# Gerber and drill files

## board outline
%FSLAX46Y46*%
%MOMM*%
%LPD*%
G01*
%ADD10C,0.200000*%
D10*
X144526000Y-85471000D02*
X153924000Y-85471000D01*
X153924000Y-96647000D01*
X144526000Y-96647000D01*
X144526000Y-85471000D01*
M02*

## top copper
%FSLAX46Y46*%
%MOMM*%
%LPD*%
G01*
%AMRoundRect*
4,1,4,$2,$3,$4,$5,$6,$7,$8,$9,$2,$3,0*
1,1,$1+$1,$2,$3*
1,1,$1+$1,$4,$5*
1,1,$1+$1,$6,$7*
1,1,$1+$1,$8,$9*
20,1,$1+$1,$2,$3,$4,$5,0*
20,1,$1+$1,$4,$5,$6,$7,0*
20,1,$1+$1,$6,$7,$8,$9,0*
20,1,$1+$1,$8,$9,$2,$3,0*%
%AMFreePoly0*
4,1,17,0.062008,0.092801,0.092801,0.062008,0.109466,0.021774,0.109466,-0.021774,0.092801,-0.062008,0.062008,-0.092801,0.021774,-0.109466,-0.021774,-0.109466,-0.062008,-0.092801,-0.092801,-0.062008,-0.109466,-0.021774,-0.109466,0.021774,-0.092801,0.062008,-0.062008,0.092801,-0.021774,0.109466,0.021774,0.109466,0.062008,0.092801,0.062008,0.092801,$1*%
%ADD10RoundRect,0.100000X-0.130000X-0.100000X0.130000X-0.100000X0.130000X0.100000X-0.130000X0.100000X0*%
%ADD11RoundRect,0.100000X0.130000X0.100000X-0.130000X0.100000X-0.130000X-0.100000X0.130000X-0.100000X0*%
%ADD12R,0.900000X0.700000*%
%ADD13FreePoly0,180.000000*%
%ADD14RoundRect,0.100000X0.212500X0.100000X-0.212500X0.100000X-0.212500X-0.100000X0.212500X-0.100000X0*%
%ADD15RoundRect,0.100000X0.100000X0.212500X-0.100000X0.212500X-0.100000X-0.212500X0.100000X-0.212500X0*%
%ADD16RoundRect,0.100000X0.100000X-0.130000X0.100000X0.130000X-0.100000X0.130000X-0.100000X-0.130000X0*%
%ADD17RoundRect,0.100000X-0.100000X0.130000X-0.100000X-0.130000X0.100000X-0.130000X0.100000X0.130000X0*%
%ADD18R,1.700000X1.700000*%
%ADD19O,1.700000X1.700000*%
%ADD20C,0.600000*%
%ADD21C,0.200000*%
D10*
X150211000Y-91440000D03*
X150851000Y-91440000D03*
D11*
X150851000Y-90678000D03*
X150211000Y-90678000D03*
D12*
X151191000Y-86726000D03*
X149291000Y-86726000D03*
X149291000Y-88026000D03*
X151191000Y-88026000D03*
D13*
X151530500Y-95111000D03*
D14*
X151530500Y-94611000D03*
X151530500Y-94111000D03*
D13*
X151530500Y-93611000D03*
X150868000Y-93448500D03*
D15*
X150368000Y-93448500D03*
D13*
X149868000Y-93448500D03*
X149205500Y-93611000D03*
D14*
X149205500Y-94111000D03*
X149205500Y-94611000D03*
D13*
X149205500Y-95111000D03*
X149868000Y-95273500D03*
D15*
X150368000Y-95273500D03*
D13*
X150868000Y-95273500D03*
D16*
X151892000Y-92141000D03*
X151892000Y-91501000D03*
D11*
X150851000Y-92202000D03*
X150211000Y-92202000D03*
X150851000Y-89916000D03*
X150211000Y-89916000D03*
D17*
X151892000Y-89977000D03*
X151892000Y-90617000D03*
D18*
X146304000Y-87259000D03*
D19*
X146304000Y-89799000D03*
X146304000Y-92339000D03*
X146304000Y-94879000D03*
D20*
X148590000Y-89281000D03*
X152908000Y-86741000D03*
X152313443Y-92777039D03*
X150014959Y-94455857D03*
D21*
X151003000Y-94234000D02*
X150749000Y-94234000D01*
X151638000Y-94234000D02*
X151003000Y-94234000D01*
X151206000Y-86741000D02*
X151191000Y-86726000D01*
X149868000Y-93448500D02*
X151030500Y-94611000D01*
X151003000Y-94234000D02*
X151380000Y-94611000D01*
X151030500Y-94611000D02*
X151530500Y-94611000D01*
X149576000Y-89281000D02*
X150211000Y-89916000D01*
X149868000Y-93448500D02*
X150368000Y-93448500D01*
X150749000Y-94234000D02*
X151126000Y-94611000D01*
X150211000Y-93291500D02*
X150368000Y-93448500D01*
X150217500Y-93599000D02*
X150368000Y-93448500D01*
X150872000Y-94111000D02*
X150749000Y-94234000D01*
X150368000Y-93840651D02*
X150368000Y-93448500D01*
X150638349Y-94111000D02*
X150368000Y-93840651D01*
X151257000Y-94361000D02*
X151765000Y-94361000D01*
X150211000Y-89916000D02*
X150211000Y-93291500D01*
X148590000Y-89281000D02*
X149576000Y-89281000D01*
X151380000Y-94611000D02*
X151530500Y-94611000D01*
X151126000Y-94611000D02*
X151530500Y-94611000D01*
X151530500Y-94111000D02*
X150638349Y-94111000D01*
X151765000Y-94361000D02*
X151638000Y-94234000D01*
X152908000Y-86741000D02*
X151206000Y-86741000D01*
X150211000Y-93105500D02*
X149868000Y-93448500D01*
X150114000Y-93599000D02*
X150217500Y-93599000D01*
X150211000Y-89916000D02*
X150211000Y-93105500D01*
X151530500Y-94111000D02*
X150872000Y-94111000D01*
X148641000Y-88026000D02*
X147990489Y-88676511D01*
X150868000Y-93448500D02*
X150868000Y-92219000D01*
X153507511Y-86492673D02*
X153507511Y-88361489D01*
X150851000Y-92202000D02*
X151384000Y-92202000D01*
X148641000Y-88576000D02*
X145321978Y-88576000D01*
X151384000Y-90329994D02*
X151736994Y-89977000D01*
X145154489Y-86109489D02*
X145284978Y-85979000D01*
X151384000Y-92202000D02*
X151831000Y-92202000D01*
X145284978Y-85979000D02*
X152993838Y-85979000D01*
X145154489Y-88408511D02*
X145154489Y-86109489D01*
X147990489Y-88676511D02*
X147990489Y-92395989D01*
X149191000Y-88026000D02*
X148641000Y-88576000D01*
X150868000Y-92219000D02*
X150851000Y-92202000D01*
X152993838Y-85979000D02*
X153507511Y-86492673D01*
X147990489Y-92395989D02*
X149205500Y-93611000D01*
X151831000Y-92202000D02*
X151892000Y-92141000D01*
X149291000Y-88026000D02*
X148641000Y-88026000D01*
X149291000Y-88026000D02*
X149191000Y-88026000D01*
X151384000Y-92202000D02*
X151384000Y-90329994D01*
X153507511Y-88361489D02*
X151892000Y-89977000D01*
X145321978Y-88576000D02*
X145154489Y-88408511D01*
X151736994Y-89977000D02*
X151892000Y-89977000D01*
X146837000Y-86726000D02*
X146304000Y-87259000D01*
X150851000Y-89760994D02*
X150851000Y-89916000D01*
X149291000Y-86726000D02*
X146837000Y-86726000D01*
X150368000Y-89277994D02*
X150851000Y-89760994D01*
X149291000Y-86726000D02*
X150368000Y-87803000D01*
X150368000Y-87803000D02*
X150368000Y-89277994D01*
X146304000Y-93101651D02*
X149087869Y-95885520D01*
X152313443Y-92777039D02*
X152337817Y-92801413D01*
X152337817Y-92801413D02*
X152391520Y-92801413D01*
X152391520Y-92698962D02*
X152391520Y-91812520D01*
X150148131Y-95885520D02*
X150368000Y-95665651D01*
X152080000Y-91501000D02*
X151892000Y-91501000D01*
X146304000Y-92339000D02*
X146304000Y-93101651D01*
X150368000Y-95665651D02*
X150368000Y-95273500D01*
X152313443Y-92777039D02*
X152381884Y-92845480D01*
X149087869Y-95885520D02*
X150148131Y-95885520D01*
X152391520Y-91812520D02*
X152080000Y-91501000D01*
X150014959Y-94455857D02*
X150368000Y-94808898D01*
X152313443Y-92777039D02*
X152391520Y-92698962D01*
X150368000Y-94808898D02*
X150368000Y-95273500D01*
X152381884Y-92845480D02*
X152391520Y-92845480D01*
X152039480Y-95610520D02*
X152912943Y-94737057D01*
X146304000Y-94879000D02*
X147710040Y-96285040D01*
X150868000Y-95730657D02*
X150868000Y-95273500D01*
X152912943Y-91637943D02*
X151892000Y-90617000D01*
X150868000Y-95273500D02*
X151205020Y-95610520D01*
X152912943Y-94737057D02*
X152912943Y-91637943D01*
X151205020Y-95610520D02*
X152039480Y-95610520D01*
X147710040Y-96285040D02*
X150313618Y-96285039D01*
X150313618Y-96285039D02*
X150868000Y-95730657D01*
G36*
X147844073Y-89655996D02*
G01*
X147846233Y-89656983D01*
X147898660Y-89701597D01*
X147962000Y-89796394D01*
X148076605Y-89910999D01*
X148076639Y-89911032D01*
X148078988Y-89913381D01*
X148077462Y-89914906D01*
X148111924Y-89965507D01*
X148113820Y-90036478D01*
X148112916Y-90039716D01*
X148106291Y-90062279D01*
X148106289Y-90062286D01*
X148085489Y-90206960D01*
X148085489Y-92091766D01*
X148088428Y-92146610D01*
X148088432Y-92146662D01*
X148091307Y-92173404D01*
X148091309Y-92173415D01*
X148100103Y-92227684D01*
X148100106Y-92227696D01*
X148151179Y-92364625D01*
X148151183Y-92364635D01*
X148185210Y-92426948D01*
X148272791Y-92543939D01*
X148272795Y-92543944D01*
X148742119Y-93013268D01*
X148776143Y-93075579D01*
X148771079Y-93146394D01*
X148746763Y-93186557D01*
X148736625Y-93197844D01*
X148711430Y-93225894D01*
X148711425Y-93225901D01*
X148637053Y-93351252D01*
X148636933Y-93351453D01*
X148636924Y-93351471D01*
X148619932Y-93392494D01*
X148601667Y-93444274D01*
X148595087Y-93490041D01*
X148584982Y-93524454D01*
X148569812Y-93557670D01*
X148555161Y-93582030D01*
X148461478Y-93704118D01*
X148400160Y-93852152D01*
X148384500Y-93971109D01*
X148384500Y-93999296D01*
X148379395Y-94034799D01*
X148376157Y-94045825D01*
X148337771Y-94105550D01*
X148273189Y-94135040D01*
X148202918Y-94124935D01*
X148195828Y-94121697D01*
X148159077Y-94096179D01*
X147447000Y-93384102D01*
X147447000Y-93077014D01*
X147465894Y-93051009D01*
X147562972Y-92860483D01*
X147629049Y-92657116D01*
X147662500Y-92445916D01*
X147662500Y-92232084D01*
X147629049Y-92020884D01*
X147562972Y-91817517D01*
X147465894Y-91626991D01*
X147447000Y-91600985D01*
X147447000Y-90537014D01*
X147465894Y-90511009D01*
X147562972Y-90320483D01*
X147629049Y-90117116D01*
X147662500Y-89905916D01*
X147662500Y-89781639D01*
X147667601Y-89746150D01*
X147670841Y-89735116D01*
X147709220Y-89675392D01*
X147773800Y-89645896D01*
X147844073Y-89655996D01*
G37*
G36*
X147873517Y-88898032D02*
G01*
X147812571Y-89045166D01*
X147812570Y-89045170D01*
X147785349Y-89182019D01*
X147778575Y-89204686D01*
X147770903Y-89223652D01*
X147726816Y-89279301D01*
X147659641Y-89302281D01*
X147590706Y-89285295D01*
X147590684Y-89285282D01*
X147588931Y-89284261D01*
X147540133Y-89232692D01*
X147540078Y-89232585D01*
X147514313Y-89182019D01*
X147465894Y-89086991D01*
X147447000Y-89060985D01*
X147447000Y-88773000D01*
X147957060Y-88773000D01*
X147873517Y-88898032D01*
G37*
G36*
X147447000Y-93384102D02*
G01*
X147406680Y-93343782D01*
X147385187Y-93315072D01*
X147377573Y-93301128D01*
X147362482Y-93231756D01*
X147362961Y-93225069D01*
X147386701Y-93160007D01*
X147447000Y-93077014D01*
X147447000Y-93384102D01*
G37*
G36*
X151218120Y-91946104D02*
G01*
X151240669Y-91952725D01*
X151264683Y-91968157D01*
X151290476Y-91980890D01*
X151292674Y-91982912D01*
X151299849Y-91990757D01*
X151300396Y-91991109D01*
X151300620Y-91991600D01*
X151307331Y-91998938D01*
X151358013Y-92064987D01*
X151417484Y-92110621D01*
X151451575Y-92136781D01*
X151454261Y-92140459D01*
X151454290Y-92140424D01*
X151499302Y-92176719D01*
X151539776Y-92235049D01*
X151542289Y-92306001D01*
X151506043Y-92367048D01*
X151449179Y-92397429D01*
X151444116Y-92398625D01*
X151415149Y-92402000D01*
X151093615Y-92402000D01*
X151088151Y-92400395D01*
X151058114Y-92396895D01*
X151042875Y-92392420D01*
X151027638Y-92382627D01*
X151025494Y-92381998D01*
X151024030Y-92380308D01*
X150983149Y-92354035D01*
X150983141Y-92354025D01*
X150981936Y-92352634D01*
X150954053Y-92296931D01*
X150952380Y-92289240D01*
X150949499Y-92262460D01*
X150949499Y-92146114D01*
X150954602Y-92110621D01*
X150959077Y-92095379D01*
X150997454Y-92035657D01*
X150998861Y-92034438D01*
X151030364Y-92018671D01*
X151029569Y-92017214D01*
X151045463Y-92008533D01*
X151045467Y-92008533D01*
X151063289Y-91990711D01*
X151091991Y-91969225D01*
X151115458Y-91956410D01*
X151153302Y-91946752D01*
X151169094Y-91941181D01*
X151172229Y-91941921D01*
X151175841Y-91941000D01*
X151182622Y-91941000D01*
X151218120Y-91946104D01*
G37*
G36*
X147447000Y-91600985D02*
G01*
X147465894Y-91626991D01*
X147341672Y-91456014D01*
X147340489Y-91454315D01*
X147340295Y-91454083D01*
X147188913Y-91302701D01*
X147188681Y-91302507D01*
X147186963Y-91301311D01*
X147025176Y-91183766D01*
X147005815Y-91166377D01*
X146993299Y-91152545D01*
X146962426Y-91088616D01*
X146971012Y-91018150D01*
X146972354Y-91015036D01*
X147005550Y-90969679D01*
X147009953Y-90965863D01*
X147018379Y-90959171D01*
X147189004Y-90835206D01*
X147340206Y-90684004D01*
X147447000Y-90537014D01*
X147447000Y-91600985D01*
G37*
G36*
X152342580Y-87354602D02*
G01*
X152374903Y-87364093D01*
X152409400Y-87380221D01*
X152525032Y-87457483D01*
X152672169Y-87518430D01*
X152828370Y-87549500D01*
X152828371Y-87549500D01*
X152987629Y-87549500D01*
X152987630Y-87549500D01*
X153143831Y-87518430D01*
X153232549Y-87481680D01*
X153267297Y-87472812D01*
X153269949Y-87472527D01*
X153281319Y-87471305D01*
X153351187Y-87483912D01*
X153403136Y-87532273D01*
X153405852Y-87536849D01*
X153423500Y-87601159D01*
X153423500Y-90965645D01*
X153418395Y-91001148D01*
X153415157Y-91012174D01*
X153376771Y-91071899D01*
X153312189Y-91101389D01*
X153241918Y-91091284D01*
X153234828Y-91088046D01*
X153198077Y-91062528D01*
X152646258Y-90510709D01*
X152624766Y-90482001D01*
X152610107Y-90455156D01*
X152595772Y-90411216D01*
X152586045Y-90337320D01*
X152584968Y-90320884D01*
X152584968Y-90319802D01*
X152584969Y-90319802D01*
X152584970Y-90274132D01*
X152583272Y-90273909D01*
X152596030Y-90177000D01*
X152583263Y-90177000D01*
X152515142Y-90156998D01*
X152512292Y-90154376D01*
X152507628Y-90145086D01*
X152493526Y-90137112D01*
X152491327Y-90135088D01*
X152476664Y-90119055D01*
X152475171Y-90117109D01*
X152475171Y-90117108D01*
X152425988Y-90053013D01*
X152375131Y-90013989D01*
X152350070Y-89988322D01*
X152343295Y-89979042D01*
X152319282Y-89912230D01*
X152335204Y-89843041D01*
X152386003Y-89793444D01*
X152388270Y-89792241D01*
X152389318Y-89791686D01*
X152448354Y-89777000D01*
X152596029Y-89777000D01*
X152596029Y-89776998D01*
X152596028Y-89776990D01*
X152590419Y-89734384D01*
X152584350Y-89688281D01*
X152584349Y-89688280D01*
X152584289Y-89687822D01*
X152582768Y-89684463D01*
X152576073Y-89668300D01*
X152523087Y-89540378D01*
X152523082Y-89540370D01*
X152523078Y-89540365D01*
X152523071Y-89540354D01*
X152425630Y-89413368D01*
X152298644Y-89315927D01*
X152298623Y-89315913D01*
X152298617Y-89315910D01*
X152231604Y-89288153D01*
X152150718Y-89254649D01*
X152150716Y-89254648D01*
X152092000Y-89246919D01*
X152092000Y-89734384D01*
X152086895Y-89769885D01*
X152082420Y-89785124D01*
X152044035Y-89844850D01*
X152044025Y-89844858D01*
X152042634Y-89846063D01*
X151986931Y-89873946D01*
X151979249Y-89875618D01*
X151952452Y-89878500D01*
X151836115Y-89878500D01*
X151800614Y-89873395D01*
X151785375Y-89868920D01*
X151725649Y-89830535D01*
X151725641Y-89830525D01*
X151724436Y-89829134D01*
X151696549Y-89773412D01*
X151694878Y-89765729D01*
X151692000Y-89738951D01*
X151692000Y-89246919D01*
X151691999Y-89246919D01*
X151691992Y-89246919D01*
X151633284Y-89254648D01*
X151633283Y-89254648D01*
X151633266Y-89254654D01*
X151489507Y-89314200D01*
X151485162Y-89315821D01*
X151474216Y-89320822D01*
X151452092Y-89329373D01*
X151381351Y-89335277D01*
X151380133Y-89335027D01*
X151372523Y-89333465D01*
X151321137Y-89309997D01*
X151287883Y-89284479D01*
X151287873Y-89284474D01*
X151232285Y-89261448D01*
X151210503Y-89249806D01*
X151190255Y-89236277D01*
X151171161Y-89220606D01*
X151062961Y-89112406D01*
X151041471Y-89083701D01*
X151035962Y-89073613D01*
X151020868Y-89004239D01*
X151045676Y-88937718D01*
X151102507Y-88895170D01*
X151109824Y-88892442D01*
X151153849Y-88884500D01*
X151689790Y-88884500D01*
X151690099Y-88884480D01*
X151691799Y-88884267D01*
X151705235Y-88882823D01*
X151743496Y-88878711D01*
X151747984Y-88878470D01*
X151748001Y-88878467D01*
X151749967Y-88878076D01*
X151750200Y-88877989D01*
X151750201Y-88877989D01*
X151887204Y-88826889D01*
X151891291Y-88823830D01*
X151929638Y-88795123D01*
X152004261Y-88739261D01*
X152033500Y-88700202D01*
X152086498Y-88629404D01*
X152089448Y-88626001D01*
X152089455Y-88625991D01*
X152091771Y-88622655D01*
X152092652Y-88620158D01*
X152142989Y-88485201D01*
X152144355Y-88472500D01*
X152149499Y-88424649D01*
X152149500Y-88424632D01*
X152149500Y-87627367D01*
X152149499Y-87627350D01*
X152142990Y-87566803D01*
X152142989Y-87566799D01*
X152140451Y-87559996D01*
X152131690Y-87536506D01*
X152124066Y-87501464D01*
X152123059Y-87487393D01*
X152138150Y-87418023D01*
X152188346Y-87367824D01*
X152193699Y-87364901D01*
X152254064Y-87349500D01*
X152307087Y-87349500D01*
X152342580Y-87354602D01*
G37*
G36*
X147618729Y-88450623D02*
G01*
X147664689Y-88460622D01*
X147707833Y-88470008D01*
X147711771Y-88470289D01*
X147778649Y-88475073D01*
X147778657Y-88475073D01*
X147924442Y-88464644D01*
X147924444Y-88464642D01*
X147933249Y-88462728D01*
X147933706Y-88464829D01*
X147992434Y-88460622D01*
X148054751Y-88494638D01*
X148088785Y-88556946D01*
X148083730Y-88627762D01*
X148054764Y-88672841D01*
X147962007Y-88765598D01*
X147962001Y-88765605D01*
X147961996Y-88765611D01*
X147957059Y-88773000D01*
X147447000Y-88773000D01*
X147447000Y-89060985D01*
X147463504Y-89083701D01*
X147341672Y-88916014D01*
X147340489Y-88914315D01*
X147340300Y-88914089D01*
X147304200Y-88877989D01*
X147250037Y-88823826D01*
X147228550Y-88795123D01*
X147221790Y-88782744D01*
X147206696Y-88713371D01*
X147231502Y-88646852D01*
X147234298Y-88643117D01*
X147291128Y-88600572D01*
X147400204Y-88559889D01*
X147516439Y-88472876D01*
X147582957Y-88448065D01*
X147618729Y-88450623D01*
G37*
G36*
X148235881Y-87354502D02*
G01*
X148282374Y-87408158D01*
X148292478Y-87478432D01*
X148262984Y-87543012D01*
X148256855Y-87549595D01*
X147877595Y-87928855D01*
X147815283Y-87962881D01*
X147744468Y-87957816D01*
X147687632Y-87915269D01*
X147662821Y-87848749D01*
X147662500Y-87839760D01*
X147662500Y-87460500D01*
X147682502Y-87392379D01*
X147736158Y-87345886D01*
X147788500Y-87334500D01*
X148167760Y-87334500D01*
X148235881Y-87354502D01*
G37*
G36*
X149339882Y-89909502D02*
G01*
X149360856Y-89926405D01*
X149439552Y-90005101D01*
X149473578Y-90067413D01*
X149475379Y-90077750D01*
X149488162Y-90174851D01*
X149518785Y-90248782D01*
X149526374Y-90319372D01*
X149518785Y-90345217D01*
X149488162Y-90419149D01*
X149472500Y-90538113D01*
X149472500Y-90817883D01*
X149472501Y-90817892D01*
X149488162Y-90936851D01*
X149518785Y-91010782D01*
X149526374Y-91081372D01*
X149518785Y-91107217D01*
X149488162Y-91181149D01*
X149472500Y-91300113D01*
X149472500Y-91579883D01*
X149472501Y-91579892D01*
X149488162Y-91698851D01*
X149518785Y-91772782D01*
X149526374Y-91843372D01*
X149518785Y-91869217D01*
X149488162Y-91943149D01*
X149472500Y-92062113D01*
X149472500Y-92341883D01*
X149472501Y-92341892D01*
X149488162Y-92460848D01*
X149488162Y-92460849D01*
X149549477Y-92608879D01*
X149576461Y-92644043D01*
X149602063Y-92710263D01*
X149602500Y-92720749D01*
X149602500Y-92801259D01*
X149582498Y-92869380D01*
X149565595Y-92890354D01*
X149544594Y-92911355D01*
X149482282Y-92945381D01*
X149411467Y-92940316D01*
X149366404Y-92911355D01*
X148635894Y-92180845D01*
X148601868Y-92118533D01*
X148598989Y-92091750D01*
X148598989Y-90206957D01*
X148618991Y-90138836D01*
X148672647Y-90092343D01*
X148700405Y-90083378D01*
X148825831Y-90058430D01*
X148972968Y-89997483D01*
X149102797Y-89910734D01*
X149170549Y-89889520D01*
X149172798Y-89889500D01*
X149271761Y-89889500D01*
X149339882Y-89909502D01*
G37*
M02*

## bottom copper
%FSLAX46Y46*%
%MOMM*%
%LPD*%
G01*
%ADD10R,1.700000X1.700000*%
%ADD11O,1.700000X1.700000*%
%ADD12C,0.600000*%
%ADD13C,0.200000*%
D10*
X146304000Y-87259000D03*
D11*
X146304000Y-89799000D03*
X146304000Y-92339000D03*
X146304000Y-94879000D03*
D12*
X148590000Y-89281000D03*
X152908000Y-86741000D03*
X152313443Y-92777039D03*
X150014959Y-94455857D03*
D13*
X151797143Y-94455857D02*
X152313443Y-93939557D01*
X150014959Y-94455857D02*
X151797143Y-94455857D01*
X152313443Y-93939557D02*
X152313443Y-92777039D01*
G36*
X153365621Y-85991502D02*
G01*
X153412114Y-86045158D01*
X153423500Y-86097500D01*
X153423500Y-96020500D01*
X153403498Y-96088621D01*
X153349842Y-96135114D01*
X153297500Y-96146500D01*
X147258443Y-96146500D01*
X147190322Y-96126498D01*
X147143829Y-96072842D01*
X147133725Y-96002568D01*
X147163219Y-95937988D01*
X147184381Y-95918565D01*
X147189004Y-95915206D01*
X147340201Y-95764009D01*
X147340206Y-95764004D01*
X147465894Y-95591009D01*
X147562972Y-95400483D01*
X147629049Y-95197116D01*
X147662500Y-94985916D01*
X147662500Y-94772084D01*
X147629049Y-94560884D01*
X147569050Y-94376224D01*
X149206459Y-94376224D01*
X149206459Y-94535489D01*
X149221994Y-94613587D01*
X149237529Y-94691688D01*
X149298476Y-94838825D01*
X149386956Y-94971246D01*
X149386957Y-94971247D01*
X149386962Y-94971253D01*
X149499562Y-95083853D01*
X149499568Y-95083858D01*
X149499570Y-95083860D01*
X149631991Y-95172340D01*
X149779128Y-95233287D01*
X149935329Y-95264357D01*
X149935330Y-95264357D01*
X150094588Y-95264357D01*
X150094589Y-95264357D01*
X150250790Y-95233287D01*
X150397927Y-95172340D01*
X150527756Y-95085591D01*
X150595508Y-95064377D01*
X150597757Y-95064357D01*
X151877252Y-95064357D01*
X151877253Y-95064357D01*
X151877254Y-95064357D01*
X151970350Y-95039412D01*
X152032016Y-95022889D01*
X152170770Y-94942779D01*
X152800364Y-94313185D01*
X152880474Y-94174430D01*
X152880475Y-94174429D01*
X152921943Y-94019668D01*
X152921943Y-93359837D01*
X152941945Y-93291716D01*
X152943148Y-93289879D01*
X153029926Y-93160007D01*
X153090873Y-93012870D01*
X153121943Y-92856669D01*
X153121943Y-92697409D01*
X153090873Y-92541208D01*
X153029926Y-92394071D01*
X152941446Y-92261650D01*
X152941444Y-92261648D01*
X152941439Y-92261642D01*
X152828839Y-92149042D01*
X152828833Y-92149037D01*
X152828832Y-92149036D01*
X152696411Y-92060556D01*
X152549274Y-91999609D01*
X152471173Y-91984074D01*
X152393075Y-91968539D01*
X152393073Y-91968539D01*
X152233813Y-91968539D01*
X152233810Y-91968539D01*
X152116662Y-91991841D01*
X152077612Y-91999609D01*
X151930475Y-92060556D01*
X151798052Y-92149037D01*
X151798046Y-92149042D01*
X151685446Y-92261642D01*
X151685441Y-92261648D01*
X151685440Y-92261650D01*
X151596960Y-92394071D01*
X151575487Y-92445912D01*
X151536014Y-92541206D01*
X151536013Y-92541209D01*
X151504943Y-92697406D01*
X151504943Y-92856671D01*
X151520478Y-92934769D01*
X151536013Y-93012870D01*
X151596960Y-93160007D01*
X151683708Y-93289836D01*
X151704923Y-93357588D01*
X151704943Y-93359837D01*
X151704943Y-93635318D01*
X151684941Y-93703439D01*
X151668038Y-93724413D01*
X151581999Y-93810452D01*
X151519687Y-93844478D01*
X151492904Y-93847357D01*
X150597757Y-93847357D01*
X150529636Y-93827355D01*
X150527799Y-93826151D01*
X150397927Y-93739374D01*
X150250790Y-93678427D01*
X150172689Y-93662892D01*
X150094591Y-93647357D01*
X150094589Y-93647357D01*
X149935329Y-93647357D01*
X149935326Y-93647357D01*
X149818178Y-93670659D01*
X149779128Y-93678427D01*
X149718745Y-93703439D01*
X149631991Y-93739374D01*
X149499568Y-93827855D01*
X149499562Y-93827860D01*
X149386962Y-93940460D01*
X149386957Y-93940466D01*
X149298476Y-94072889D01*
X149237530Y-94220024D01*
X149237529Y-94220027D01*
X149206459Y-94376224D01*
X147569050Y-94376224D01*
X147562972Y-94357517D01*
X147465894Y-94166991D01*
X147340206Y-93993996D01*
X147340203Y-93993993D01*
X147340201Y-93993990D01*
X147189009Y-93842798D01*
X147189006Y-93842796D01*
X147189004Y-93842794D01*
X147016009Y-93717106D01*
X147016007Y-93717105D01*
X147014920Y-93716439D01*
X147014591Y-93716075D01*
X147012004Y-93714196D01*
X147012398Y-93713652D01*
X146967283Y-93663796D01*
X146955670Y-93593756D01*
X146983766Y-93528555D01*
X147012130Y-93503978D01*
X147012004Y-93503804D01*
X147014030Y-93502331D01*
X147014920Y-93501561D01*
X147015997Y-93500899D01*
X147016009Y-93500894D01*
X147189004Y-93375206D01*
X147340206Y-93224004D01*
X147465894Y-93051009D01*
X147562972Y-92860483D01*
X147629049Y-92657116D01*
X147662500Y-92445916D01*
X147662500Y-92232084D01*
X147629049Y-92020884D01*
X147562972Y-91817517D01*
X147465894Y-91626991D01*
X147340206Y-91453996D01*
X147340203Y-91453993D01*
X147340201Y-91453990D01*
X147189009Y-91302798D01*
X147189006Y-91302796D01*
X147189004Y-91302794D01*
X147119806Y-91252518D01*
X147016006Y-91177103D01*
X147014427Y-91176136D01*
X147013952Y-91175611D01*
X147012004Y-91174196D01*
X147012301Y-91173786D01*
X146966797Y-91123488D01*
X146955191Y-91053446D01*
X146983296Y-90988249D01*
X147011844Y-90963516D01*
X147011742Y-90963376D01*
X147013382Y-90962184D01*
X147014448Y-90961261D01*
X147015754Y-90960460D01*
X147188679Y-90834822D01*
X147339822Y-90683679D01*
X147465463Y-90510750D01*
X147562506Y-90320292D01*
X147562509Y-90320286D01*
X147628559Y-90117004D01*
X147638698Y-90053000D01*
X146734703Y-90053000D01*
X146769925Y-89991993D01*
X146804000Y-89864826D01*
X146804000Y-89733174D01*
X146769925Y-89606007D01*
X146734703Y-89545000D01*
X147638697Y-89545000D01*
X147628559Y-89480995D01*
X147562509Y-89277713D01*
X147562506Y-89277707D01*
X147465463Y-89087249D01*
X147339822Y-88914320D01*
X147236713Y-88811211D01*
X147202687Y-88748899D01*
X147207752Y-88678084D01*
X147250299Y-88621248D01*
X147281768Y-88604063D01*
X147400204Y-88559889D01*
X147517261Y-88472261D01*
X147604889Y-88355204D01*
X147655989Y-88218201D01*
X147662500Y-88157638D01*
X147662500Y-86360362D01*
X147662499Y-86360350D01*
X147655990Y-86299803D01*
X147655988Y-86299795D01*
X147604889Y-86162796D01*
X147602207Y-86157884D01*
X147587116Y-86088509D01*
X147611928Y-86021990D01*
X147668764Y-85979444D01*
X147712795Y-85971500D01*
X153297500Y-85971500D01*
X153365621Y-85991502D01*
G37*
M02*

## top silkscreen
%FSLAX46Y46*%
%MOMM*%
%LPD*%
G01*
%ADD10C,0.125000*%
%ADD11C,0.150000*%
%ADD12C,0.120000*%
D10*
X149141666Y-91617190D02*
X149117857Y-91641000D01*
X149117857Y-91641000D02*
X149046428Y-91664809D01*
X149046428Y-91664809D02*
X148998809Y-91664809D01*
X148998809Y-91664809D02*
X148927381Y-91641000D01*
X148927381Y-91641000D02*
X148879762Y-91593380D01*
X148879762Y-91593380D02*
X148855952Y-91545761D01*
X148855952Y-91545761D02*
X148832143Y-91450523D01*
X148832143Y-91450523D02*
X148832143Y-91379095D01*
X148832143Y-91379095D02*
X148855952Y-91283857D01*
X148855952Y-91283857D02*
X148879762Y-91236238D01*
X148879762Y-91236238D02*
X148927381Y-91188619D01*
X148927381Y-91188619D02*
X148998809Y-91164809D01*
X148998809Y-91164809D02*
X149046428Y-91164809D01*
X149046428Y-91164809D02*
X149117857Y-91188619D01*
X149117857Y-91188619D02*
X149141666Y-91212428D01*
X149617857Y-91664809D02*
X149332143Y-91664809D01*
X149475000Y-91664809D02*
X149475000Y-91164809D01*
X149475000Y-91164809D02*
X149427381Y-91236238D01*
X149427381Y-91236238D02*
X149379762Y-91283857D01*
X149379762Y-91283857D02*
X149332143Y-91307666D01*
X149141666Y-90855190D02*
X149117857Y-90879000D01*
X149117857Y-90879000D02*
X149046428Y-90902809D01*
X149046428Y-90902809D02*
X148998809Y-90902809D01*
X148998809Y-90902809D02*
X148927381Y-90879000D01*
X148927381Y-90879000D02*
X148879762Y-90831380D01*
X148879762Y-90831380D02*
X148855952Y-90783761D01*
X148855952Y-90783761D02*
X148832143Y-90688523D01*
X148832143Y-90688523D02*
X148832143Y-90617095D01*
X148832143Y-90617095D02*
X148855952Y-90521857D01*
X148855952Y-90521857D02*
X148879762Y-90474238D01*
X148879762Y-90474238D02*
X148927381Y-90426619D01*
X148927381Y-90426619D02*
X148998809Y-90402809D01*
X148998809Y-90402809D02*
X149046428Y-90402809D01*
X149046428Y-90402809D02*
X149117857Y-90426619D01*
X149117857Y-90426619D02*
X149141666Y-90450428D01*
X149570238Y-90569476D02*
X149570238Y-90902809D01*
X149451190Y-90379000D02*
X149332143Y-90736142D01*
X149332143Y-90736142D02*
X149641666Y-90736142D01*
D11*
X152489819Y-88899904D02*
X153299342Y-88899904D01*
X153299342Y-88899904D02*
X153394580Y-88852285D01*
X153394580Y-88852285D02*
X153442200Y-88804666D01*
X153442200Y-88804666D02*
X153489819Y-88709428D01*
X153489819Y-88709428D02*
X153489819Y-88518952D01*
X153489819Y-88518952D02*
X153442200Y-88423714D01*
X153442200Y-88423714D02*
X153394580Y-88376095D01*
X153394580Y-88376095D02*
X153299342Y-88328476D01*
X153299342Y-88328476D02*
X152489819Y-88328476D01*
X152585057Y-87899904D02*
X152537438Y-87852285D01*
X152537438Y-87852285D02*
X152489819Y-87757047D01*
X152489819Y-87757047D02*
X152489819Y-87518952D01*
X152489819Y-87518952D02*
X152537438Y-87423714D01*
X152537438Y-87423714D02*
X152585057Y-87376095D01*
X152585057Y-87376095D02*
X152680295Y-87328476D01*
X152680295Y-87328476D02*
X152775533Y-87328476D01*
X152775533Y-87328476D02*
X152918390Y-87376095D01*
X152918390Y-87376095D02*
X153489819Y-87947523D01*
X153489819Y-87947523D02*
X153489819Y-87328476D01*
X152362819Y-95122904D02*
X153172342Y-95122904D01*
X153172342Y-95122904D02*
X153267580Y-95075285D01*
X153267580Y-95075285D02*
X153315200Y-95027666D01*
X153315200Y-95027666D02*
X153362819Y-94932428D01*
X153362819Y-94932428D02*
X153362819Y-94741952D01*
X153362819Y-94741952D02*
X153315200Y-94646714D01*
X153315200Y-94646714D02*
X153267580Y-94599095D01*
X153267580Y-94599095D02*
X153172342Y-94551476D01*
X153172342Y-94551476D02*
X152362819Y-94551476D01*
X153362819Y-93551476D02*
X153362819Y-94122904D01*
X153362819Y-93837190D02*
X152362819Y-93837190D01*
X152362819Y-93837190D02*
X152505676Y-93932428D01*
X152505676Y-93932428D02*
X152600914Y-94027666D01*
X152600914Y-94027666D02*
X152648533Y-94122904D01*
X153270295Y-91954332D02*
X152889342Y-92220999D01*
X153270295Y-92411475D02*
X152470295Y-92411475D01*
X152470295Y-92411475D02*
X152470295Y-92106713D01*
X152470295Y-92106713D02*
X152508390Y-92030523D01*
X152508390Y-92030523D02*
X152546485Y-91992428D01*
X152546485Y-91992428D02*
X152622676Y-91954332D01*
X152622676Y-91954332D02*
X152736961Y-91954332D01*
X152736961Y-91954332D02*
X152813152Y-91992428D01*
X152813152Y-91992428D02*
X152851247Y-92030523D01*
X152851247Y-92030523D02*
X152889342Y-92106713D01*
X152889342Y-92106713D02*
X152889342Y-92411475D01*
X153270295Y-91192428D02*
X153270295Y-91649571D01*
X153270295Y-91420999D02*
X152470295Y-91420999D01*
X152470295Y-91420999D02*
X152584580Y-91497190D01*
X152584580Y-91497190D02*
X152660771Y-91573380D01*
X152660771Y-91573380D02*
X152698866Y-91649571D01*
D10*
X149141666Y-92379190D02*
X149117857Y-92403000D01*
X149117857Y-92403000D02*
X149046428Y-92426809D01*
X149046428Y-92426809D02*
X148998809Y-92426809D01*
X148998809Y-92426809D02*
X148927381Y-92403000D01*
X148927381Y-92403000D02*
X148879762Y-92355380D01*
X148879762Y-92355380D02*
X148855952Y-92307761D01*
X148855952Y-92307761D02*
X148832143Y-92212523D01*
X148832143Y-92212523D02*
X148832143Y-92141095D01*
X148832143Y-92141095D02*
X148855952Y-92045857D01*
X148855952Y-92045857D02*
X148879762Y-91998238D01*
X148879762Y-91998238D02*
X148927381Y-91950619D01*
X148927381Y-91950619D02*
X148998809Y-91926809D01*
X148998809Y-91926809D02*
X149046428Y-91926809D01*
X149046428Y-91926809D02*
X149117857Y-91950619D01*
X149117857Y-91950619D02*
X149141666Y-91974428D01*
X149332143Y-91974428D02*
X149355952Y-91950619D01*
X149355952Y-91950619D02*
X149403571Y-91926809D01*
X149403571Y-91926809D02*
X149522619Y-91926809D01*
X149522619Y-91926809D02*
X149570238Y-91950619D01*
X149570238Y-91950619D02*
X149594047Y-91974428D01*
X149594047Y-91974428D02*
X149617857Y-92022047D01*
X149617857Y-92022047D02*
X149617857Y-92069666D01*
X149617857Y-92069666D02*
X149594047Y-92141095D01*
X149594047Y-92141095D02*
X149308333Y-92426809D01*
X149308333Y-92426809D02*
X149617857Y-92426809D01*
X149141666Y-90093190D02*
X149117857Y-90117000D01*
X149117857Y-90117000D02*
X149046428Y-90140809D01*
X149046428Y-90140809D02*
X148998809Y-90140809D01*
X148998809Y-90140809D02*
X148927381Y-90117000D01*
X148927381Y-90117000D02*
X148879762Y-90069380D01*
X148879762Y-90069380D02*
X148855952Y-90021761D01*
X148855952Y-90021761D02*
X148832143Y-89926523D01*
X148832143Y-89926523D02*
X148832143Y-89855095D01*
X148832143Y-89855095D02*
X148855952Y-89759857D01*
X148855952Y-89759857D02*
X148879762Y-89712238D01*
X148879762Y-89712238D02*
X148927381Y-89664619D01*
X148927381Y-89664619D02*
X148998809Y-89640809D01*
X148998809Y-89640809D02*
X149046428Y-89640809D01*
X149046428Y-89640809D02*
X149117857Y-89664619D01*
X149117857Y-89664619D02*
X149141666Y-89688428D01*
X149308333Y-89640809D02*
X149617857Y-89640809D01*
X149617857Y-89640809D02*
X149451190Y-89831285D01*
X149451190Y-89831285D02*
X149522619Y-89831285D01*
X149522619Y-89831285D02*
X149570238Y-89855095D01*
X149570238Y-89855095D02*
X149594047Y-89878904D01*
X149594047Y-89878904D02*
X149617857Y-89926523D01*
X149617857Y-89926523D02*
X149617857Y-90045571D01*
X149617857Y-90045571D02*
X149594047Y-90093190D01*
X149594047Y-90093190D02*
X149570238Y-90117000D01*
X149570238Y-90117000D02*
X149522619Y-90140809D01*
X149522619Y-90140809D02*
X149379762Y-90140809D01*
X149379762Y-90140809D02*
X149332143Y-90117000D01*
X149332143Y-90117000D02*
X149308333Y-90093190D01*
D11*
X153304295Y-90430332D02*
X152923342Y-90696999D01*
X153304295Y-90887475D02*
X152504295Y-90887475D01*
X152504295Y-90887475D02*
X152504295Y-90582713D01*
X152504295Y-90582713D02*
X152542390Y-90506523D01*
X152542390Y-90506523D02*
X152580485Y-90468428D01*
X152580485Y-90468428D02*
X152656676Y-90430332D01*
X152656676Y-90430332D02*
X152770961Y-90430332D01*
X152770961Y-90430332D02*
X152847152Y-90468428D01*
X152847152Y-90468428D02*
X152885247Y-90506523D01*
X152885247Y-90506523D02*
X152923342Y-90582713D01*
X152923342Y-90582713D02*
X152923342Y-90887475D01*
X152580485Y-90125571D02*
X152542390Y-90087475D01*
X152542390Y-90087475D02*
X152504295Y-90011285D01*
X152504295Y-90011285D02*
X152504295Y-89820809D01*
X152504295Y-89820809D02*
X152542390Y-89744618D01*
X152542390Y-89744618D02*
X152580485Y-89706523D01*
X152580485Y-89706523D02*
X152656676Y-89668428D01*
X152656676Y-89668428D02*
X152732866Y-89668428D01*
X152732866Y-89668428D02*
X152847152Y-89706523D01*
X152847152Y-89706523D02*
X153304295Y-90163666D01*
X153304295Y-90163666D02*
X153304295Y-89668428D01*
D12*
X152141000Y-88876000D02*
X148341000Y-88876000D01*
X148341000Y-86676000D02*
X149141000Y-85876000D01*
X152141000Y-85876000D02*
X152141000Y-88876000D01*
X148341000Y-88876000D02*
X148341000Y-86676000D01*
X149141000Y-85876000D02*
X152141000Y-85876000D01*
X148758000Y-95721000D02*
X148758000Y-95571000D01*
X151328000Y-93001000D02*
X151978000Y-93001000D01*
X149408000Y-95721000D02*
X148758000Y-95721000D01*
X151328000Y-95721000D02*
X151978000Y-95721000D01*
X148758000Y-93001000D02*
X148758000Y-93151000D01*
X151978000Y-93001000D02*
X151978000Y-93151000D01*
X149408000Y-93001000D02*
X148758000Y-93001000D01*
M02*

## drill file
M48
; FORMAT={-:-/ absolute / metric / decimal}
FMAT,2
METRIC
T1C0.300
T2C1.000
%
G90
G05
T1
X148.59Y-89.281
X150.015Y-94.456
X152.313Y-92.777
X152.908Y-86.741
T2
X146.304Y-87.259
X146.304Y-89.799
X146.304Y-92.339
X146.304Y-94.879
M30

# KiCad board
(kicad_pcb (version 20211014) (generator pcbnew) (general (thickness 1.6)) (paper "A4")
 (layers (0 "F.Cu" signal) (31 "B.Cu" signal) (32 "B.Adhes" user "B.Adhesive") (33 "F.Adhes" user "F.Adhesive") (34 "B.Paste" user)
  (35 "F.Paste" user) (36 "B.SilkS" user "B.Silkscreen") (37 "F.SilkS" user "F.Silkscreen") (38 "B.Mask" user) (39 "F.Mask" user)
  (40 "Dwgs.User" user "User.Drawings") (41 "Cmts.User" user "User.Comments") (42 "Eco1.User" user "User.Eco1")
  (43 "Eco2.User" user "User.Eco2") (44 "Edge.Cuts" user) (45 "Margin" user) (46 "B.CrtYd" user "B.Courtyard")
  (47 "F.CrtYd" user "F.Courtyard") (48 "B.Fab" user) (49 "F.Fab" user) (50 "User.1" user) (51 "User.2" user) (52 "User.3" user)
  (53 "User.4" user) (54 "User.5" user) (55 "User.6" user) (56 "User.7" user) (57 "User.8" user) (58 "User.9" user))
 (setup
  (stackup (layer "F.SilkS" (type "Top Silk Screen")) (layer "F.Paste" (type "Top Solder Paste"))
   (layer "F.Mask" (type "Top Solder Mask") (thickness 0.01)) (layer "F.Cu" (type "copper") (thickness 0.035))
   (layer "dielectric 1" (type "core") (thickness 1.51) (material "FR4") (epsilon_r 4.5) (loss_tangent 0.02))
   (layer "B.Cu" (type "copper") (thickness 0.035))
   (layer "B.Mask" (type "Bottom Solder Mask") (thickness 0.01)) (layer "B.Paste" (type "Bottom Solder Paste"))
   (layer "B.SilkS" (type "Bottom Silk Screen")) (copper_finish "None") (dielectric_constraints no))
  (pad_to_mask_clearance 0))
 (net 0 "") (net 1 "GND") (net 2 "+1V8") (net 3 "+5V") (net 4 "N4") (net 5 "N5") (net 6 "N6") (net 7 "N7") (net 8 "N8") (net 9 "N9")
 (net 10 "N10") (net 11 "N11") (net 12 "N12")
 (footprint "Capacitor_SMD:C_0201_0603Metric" (layer "F.Cu") (at 150.531 91.44)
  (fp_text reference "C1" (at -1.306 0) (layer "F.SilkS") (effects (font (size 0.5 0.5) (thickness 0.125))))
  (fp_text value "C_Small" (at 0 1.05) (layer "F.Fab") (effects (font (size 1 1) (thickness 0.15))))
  (pad "" smd roundrect (at -0.345 0) (size 0.318 0.36) (layers "F.Paste") (roundrect_rratio 0.25))
  (pad "" smd roundrect (at 0.345 0) (size 0.318 0.36) (layers "F.Paste") (roundrect_rratio 0.25))
  (pad "1" smd roundrect (at -0.32 0) (size 0.46 0.4) (layers "F.Cu" "F.Mask") (roundrect_rratio 0.25) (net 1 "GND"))
  (pad "2" smd roundrect (at 0.32 0) (size 0.46 0.4) (layers "F.Cu" "F.Mask") (roundrect_rratio 0.25) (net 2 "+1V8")))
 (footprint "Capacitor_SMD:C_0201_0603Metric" (layer "F.Cu") (at 150.531 90.678 180)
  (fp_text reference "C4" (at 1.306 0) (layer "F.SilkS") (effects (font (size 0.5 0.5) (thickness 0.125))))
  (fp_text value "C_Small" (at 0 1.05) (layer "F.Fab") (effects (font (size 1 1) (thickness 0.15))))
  (pad "" smd roundrect (at -0.345 0 180) (size 0.318 0.36) (layers "F.Paste") (roundrect_rratio 0.25))
  (pad "" smd roundrect (at 0.345 0 180) (size 0.318 0.36) (layers "F.Paste") (roundrect_rratio 0.25))
  (pad "1" smd roundrect (at -0.32 0 180) (size 0.46 0.4) (layers "F.Cu" "F.Mask") (roundrect_rratio 0.25) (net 2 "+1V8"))
  (pad "2" smd roundrect (at 0.32 0 180) (size 0.46 0.4) (layers "F.Cu" "F.Mask") (roundrect_rratio 0.25) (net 1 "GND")))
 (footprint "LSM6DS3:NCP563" (layer "F.Cu") (at 150.241 87.376 -90)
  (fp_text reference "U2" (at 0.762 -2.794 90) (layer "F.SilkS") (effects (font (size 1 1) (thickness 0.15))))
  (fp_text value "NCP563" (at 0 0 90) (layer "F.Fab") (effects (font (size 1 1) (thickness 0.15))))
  (fp_line (start 1.5 -1.9) (end 1.5 1.9) (layer "F.SilkS") (width 0.12))
  (fp_line (start -0.7 1.9) (end -1.5 1.1) (layer "F.SilkS") (width 0.12))
  (fp_line (start -1.5 -1.9) (end 1.5 -1.9) (layer "F.SilkS") (width 0.12))
  (fp_line (start 1.5 1.9) (end -0.7 1.9) (layer "F.SilkS") (width 0.12))
  (fp_line (start -1.5 1.1) (end -1.5 -1.9) (layer "F.SilkS") (width 0.12))
  (pad "1" smd rect (at -0.65 -0.95 270) (size 0.7 0.9) (layers "F.Cu" "F.Paste" "F.Mask") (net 1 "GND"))
  (pad "2" smd rect (at -0.65 0.95 270) (size 0.7 0.9) (layers "F.Cu" "F.Paste" "F.Mask") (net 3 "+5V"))
  (pad "3" smd rect (at 0.65 0.95 270) (size 0.7 0.9) (layers "F.Cu" "F.Paste" "F.Mask") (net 2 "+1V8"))
  (pad "4" smd rect (at 0.65 -0.95 270) (size 0.7 0.9) (layers "F.Cu" "F.Paste" "F.Mask") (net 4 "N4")))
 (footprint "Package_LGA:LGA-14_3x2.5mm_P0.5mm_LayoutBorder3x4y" (layer "F.Cu") (at 150.368 94.361 180)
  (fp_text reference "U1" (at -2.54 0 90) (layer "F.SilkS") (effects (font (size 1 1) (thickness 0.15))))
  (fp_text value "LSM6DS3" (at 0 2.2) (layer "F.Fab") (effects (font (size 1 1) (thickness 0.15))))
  (fp_line (start 1.61 -1.36) (end 1.61 -1.21) (layer "F.SilkS") (width 0.12))
  (fp_line (start -0.96 1.36) (end -1.61 1.36) (layer "F.SilkS") (width 0.12))
  (fp_line (start 0.96 -1.36) (end 1.61 -1.36) (layer "F.SilkS") (width 0.12))
  (fp_line (start -0.96 -1.36) (end -1.61 -1.36) (layer "F.SilkS") (width 0.12))
  (fp_line (start 1.61 1.36) (end 1.61 1.21) (layer "F.SilkS") (width 0.12))
  (fp_line (start -1.61 1.36) (end -1.61 1.21) (layer "F.SilkS") (width 0.12))
  (fp_line (start 0.96 1.36) (end 1.61 1.36) (layer "F.SilkS") (width 0.12))
  (pad "1" smd custom (at -1.1625 -0.75 180) (size 0.223223 0.223223) (layers "F.Cu" "F.Paste" "F.Mask") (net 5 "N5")
   (options (clearance outline) (anchor circle)) (primitives))
  (pad "2" smd roundrect (at -1.1625 -0.25 180) (size 0.625 0.4) (layers "F.Cu" "F.Paste" "F.Mask") (roundrect_rratio 0.25) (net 1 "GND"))
  (pad "3" smd roundrect (at -1.1625 0.25 180) (size 0.625 0.4) (layers "F.Cu" "F.Paste" "F.Mask") (roundrect_rratio 0.25) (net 1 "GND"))
  (pad "4" smd custom (at -1.1625 0.75 180) (size 0.223223 0.223223) (layers "F.Cu" "F.Paste" "F.Mask") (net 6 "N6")
   (options (clearance outline) (anchor circle)) (primitives))
  (pad "5" smd custom (at -0.5 0.9125 180) (size 0.223223 0.223223) (layers "F.Cu" "F.Paste" "F.Mask") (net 2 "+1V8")
   (options (clearance outline) (anchor circle)) (primitives))
  (pad "6" smd roundrect (at 0 0.9125 180) (size 0.4 0.625) (layers "F.Cu" "F.Paste" "F.Mask") (roundrect_rratio 0.25) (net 1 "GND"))
  (pad "7" smd custom (at 0.5 0.9125 180) (size 0.223223 0.223223) (layers "F.Cu" "F.Paste" "F.Mask") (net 1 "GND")
   (options (clearance outline) (anchor circle)) (primitives))
  (pad "8" smd custom (at 1.1625 0.75 180) (size 0.223223 0.223223) (layers "F.Cu" "F.Paste" "F.Mask") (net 2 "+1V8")
   (options (clearance outline) (anchor circle)) (primitives))
  (pad "9" smd roundrect (at 1.1625 0.25 180) (size 0.625 0.4) (layers "F.Cu" "F.Paste" "F.Mask") (roundrect_rratio 0.25) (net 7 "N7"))
  (pad "10" smd roundrect (at 1.1625 -0.25 180) (size 0.625 0.4) (layers "F.Cu" "F.Paste" "F.Mask") (roundrect_rratio 0.25) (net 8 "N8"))
  (pad "11" smd custom (at 1.1625 -0.75 180) (size 0.223223 0.223223) (layers "F.Cu" "F.Paste" "F.Mask") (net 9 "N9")
   (options (clearance outline) (anchor circle)) (primitives))
  (pad "12" smd custom (at 0.5 -0.9125 180) (size 0.223223 0.223223) (layers "F.Cu" "F.Paste" "F.Mask") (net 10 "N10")
   (options (clearance outline) (anchor circle)) (primitives))
  (pad "13" smd roundrect (at 0 -0.9125 180) (size 0.4 0.625) (layers "F.Cu" "F.Paste" "F.Mask") (roundrect_rratio 0.25) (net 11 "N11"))
  (pad "14" smd custom (at -0.5 -0.9125 180) (size 0.223223 0.223223) (layers "F.Cu" "F.Paste" "F.Mask") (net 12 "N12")
   (options (clearance outline) (anchor circle)) (primitives)))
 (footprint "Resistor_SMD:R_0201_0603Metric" (layer "F.Cu") (at 151.892 91.821 90)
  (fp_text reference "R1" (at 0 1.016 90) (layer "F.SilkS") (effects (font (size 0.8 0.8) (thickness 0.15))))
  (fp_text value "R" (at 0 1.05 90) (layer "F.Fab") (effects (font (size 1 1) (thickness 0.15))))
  (pad "" smd roundrect (at -0.345 0 90) (size 0.318 0.36) (layers "F.Paste") (roundrect_rratio 0.25))
  (pad "" smd roundrect (at 0.345 0 90) (size 0.318 0.36) (layers "F.Paste") (roundrect_rratio 0.25))
  (pad "1" smd roundrect (at -0.32 0 90) (size 0.46 0.4) (layers "F.Cu" "F.Mask") (roundrect_rratio 0.25) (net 2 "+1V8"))
  (pad "2" smd roundrect (at 0.32 0 90) (size 0.46 0.4) (layers "F.Cu" "F.Mask") (roundrect_rratio 0.25) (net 11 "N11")))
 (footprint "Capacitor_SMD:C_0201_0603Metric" (layer "F.Cu") (at 150.531 92.202 180)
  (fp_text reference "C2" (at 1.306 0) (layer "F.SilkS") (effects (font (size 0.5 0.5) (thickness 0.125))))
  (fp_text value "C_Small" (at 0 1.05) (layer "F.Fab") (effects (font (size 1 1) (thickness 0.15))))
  (pad "" smd roundrect (at 0.345 0 180) (size 0.318 0.36) (layers "F.Paste") (roundrect_rratio 0.25))
  (pad "" smd roundrect (at -0.345 0 180) (size 0.318 0.36) (layers "F.Paste") (roundrect_rratio 0.25))
  (pad "1" smd roundrect (at -0.32 0 180) (size 0.46 0.4) (layers "F.Cu" "F.Mask") (roundrect_rratio 0.25) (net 2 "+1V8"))
  (pad "2" smd roundrect (at 0.32 0 180) (size 0.46 0.4) (layers "F.Cu" "F.Mask") (roundrect_rratio 0.25) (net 1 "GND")))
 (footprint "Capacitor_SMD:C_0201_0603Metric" (layer "F.Cu") (at 150.531 89.916 180)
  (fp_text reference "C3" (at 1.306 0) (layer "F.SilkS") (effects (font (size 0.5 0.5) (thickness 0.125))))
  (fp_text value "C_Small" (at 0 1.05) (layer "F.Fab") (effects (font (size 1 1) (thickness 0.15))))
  (pad "" smd roundrect (at -0.345 0 180) (size 0.318 0.36) (layers "F.Paste") (roundrect_rratio 0.25))
  (pad "" smd roundrect (at 0.345 0 180) (size 0.318 0.36) (layers "F.Paste") (roundrect_rratio 0.25))
  (pad "1" smd roundrect (at -0.32 0 180) (size 0.46 0.4) (layers "F.Cu" "F.Mask") (roundrect_rratio 0.25) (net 3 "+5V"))
  (pad "2" smd roundrect (at 0.32 0 180) (size 0.46 0.4) (layers "F.Cu" "F.Mask") (roundrect_rratio 0.25) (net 1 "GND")))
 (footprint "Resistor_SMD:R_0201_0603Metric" (layer "F.Cu") (at 151.892 90.297 -90)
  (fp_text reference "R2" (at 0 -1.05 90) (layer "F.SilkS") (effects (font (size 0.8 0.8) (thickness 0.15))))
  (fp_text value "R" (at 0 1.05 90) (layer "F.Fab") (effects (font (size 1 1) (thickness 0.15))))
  (pad "" smd roundrect (at 0.345 0 270) (size 0.318 0.36) (layers "F.Paste") (roundrect_rratio 0.25))
  (pad "" smd roundrect (at -0.345 0 270) (size 0.318 0.36) (layers "F.Paste") (roundrect_rratio 0.25))
  (pad "1" smd roundrect (at -0.32 0 270) (size 0.46 0.4) (layers "F.Cu" "F.Mask") (roundrect_rratio 0.25) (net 2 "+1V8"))
  (pad "2" smd roundrect (at 0.32 0 270) (size 0.46 0.4) (layers "F.Cu" "F.Mask") (roundrect_rratio 0.25) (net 12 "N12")))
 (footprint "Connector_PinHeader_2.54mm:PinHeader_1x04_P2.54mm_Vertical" (layer "B.Cu") (at 146.304 87.259 180)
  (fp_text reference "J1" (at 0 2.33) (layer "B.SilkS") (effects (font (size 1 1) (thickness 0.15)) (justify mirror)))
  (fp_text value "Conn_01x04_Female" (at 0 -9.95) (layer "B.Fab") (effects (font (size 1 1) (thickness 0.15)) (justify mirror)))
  (pad "1" thru_hole rect (at 0 0 180) (size 1.7 1.7) (drill 1) (layers *.Cu *.Mask) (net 3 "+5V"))
  (pad "2" thru_hole oval (at 0 -2.54 180) (size 1.7 1.7) (drill 1) (layers *.Cu *.Mask) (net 1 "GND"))
  (pad "3" thru_hole oval (at 0 -5.08 180) (size 1.7 1.7) (drill 1) (layers *.Cu *.Mask) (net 11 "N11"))
  (pad "4" thru_hole oval (at 0 -7.62 180) (size 1.7 1.7) (drill 1) (layers *.Cu *.Mask) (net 12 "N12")))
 (gr_rect (start 144.526 85.471) (end 153.924 96.647) (layer "Edge.Cuts") (width 0.2) (fill none))
 (segment (start 151.003 94.234) (end 150.749 94.234) (width 0.2) (layer "F.Cu") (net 1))
 (segment (start 151.638 94.234) (end 151.003 94.234) (width 0.2) (layer "F.Cu") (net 1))
 (segment (start 151.206 86.741) (end 151.191 86.726) (width 0.2) (layer "F.Cu") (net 1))
 (segment (start 149.868 93.4485) (end 151.0305 94.611) (width 0.2) (layer "F.Cu") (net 1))
 (segment (start 151.003 94.234) (end 151.38 94.611) (width 0.2) (layer "F.Cu") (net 1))
 (segment (start 151.0305 94.611) (end 151.5305 94.611) (width 0.2) (layer "F.Cu") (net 1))
 (segment (start 149.576 89.281) (end 150.211 89.916) (width 0.2) (layer "F.Cu") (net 1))
 (segment (start 149.868 93.4485) (end 150.368 93.4485) (width 0.2) (layer "F.Cu") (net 1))
 (segment (start 150.749 94.234) (end 151.126 94.611) (width 0.2) (layer "F.Cu") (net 1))
 (segment (start 150.211 93.2915) (end 150.368 93.4485) (width 0.2) (layer "F.Cu") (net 1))
 (segment (start 150.2175 93.599) (end 150.368 93.4485) (width 0.2) (layer "F.Cu") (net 1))
 (segment (start 150.872 94.111) (end 150.749 94.234) (width 0.2) (layer "F.Cu") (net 1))
 (segment (start 150.368 93.840651) (end 150.368 93.4485) (width 0.2) (layer "F.Cu") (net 1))
 (segment (start 150.638349 94.111) (end 150.368 93.840651) (width 0.2) (layer "F.Cu") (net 1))
 (segment (start 151.257 94.361) (end 151.765 94.361) (width 0.2) (layer "F.Cu") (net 1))
 (segment (start 150.211 89.916) (end 150.211 93.2915) (width 0.2) (layer "F.Cu") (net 1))
 (segment (start 148.59 89.281) (end 149.576 89.281) (width 0.2) (layer "F.Cu") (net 1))
 (segment (start 151.38 94.611) (end 151.5305 94.611) (width 0.2) (layer "F.Cu") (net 1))
 (segment (start 151.126 94.611) (end 151.5305 94.611) (width 0.2) (layer "F.Cu") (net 1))
 (segment (start 151.5305 94.111) (end 150.638349 94.111) (width 0.2) (layer "F.Cu") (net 1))
 (segment (start 151.765 94.361) (end 151.638 94.234) (width 0.2) (layer "F.Cu") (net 1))
 (segment (start 152.908 86.741) (end 151.206 86.741) (width 0.2) (layer "F.Cu") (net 1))
 (segment (start 150.211 93.1055) (end 149.868 93.4485) (width 0.2) (layer "F.Cu") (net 1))
 (segment (start 150.114 93.599) (end 150.2175 93.599) (width 0.2) (layer "F.Cu") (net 1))
 (segment (start 150.211 89.916) (end 150.211 93.1055) (width 0.2) (layer "F.Cu") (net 1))
 (segment (start 151.5305 94.111) (end 150.872 94.111) (width 0.2) (layer "F.Cu") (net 1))
 (via (at 148.59 89.281) (size 0.6) (drill 0.3) (layers "F.Cu" "B.Cu") (free) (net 1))
 (via (at 152.908 86.741) (size 0.6) (drill 0.3) (layers "F.Cu" "B.Cu") (free) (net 1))
 (segment (start 148.641 88.026) (end 147.990489 88.676511) (width 0.2) (layer "F.Cu") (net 2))
 (segment (start 150.868 93.4485) (end 150.868 92.219) (width 0.2) (layer "F.Cu") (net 2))
 (segment (start 153.507511 86.492673) (end 153.507511 88.361489) (width 0.2) (layer "F.Cu") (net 2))
 (segment (start 150.851 92.202) (end 151.384 92.202) (width 0.2) (layer "F.Cu") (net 2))
 (segment (start 148.641 88.576) (end 145.321978 88.576) (width 0.2) (layer "F.Cu") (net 2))
 (segment (start 151.384 90.329994) (end 151.736994 89.977) (width 0.2) (layer "F.Cu") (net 2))
 (segment (start 145.154489 86.109489) (end 145.284978 85.979) (width 0.2) (layer "F.Cu") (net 2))
 (segment (start 151.384 92.202) (end 151.831 92.202) (width 0.2) (layer "F.Cu") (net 2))
 (segment (start 145.284978 85.979) (end 152.993838 85.979) (width 0.2) (layer "F.Cu") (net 2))
 (segment (start 145.154489 88.408511) (end 145.154489 86.109489) (width 0.2) (layer "F.Cu") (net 2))
 (segment (start 147.990489 88.676511) (end 147.990489 92.395989) (width 0.2) (layer "F.Cu") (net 2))
 (segment (start 149.191 88.026) (end 148.641 88.576) (width 0.2) (layer "F.Cu") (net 2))
 (segment (start 150.868 92.219) (end 150.851 92.202) (width 0.2) (layer "F.Cu") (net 2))
 (segment (start 152.993838 85.979) (end 153.507511 86.492673) (width 0.2) (layer "F.Cu") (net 2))
 (segment (start 147.990489 92.395989) (end 149.2055 93.611) (width 0.2) (layer "F.Cu") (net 2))
 (segment (start 151.831 92.202) (end 151.892 92.141) (width 0.2) (layer "F.Cu") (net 2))
 (segment (start 149.291 88.026) (end 148.641 88.026) (width 0.2) (layer "F.Cu") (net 2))
 (segment (start 149.291 88.026) (end 149.191 88.026) (width 0.2) (layer "F.Cu") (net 2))
 (segment (start 151.384 92.202) (end 151.384 90.329994) (width 0.2) (layer "F.Cu") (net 2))
 (segment (start 153.507511 88.361489) (end 151.892 89.977) (width 0.2) (layer "F.Cu") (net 2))
 (segment (start 145.321978 88.576) (end 145.154489 88.408511) (width 0.2) (layer "F.Cu") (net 2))
 (segment (start 151.736994 89.977) (end 151.892 89.977) (width 0.2) (layer "F.Cu") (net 2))
 (segment (start 146.837 86.726) (end 146.304 87.259) (width 0.2) (layer "F.Cu") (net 3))
 (segment (start 150.851 89.760994) (end 150.851 89.916) (width 0.2) (layer "F.Cu") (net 3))
 (segment (start 149.291 86.726) (end 146.837 86.726) (width 0.2) (layer "F.Cu") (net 3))
 (segment (start 150.368 89.277994) (end 150.851 89.760994) (width 0.2) (layer "F.Cu") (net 3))
 (segment (start 149.291 86.726) (end 150.368 87.803) (width 0.2) (layer "F.Cu") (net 3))
 (segment (start 150.368 87.803) (end 150.368 89.277994) (width 0.2) (layer "F.Cu") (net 3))
 (segment (start 146.304 93.101651) (end 149.087869 95.88552) (width 0.2) (layer "F.Cu") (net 11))
 (segment (start 152.313443 92.777039) (end 152.337817 92.801413) (width 0.2) (layer "F.Cu") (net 11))
 (segment (start 152.337817 92.801413) (end 152.39152 92.801413) (width 0.2) (layer "F.Cu") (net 11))
 (segment (start 152.39152 92.698962) (end 152.39152 91.81252) (width 0.2) (layer "F.Cu") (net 11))
 (segment (start 150.148131 95.88552) (end 150.368 95.665651) (width 0.2) (layer "F.Cu") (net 11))
 (segment (start 152.08 91.501) (end 151.892 91.501) (width 0.2) (layer "F.Cu") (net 11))
 (segment (start 146.304 92.339) (end 146.304 93.101651) (width 0.2) (layer "F.Cu") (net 11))
 (segment (start 150.368 95.665651) (end 150.368 95.2735) (width 0.2) (layer "F.Cu") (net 11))
 (segment (start 152.313443 92.777039) (end 152.381884 92.84548) (width 0.2) (layer "F.Cu") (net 11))
 (segment (start 149.087869 95.88552) (end 150.148131 95.88552) (width 0.2) (layer "F.Cu") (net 11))
 (segment (start 152.39152 91.81252) (end 152.08 91.501) (width 0.2) (layer "F.Cu") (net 11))
 (segment (start 150.014959 94.455857) (end 150.368 94.808898) (width 0.2) (layer "F.Cu") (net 11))
 (segment (start 152.313443 92.777039) (end 152.39152 92.698962) (width 0.2) (layer "F.Cu") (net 11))
 (segment (start 150.368 94.808898) (end 150.368 95.2735) (width 0.2) (layer "F.Cu") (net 11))
 (segment (start 152.381884 92.84548) (end 152.39152 92.84548) (width 0.2) (layer "F.Cu") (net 11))
 (via (at 152.313443 92.777039) (size 0.6) (drill 0.3) (layers "F.Cu" "B.Cu") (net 11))
 (via (at 150.014959 94.455857) (size 0.6) (drill 0.3) (layers "F.Cu" "B.Cu") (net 11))
 (segment (start 151.797143 94.455857) (end 152.313443 93.939557) (width 0.2) (layer "B.Cu") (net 11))
 (segment (start 150.014959 94.455857) (end 151.797143 94.455857) (width 0.2) (layer "B.Cu") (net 11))
 (segment (start 152.313443 93.939557) (end 152.313443 92.777039) (width 0.2) (layer "B.Cu") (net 11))
 (segment (start 152.03948 95.61052) (end 152.912943 94.737057) (width 0.2) (layer "F.Cu") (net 12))
 (segment (start 146.304 94.879) (end 147.71004 96.28504) (width 0.2) (layer "F.Cu") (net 12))
 (segment (start 150.868 95.730657) (end 150.868 95.2735) (width 0.2) (layer "F.Cu") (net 12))
 (segment (start 152.912943 91.637943) (end 151.892 90.617) (width 0.2) (layer "F.Cu") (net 12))
 (segment (start 150.868 95.2735) (end 151.20502 95.61052) (width 0.2) (layer "F.Cu") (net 12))
 (segment (start 152.912943 94.737057) (end 152.912943 91.637943) (width 0.2) (layer "F.Cu") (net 12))
 (segment (start 151.20502 95.61052) (end 152.03948 95.61052) (width 0.2) (layer "F.Cu") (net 12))
 (segment (start 147.71004 96.28504) (end 150.313618 96.285039) (width 0.2) (layer "F.Cu") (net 12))
 (segment (start 150.313618 96.285039) (end 150.868 95.730657) (width 0.2) (layer "F.Cu") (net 12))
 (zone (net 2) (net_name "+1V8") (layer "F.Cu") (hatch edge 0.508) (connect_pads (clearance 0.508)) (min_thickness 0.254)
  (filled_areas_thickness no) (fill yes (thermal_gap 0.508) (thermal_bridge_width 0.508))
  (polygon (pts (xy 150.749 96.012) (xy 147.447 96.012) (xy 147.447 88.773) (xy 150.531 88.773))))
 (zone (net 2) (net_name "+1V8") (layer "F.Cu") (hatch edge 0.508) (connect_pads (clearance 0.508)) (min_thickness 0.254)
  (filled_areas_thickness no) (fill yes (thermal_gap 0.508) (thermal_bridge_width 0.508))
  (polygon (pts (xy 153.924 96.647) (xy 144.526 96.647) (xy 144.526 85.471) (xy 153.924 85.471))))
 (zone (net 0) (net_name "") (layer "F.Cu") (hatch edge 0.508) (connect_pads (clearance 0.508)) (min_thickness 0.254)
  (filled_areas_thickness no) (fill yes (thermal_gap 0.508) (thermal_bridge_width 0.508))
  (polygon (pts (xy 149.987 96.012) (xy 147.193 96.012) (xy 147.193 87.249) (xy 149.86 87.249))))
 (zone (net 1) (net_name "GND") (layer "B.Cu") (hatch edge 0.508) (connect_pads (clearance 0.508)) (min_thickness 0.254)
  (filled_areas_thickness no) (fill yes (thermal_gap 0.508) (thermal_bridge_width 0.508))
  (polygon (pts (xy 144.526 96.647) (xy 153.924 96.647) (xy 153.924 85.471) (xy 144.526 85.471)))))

